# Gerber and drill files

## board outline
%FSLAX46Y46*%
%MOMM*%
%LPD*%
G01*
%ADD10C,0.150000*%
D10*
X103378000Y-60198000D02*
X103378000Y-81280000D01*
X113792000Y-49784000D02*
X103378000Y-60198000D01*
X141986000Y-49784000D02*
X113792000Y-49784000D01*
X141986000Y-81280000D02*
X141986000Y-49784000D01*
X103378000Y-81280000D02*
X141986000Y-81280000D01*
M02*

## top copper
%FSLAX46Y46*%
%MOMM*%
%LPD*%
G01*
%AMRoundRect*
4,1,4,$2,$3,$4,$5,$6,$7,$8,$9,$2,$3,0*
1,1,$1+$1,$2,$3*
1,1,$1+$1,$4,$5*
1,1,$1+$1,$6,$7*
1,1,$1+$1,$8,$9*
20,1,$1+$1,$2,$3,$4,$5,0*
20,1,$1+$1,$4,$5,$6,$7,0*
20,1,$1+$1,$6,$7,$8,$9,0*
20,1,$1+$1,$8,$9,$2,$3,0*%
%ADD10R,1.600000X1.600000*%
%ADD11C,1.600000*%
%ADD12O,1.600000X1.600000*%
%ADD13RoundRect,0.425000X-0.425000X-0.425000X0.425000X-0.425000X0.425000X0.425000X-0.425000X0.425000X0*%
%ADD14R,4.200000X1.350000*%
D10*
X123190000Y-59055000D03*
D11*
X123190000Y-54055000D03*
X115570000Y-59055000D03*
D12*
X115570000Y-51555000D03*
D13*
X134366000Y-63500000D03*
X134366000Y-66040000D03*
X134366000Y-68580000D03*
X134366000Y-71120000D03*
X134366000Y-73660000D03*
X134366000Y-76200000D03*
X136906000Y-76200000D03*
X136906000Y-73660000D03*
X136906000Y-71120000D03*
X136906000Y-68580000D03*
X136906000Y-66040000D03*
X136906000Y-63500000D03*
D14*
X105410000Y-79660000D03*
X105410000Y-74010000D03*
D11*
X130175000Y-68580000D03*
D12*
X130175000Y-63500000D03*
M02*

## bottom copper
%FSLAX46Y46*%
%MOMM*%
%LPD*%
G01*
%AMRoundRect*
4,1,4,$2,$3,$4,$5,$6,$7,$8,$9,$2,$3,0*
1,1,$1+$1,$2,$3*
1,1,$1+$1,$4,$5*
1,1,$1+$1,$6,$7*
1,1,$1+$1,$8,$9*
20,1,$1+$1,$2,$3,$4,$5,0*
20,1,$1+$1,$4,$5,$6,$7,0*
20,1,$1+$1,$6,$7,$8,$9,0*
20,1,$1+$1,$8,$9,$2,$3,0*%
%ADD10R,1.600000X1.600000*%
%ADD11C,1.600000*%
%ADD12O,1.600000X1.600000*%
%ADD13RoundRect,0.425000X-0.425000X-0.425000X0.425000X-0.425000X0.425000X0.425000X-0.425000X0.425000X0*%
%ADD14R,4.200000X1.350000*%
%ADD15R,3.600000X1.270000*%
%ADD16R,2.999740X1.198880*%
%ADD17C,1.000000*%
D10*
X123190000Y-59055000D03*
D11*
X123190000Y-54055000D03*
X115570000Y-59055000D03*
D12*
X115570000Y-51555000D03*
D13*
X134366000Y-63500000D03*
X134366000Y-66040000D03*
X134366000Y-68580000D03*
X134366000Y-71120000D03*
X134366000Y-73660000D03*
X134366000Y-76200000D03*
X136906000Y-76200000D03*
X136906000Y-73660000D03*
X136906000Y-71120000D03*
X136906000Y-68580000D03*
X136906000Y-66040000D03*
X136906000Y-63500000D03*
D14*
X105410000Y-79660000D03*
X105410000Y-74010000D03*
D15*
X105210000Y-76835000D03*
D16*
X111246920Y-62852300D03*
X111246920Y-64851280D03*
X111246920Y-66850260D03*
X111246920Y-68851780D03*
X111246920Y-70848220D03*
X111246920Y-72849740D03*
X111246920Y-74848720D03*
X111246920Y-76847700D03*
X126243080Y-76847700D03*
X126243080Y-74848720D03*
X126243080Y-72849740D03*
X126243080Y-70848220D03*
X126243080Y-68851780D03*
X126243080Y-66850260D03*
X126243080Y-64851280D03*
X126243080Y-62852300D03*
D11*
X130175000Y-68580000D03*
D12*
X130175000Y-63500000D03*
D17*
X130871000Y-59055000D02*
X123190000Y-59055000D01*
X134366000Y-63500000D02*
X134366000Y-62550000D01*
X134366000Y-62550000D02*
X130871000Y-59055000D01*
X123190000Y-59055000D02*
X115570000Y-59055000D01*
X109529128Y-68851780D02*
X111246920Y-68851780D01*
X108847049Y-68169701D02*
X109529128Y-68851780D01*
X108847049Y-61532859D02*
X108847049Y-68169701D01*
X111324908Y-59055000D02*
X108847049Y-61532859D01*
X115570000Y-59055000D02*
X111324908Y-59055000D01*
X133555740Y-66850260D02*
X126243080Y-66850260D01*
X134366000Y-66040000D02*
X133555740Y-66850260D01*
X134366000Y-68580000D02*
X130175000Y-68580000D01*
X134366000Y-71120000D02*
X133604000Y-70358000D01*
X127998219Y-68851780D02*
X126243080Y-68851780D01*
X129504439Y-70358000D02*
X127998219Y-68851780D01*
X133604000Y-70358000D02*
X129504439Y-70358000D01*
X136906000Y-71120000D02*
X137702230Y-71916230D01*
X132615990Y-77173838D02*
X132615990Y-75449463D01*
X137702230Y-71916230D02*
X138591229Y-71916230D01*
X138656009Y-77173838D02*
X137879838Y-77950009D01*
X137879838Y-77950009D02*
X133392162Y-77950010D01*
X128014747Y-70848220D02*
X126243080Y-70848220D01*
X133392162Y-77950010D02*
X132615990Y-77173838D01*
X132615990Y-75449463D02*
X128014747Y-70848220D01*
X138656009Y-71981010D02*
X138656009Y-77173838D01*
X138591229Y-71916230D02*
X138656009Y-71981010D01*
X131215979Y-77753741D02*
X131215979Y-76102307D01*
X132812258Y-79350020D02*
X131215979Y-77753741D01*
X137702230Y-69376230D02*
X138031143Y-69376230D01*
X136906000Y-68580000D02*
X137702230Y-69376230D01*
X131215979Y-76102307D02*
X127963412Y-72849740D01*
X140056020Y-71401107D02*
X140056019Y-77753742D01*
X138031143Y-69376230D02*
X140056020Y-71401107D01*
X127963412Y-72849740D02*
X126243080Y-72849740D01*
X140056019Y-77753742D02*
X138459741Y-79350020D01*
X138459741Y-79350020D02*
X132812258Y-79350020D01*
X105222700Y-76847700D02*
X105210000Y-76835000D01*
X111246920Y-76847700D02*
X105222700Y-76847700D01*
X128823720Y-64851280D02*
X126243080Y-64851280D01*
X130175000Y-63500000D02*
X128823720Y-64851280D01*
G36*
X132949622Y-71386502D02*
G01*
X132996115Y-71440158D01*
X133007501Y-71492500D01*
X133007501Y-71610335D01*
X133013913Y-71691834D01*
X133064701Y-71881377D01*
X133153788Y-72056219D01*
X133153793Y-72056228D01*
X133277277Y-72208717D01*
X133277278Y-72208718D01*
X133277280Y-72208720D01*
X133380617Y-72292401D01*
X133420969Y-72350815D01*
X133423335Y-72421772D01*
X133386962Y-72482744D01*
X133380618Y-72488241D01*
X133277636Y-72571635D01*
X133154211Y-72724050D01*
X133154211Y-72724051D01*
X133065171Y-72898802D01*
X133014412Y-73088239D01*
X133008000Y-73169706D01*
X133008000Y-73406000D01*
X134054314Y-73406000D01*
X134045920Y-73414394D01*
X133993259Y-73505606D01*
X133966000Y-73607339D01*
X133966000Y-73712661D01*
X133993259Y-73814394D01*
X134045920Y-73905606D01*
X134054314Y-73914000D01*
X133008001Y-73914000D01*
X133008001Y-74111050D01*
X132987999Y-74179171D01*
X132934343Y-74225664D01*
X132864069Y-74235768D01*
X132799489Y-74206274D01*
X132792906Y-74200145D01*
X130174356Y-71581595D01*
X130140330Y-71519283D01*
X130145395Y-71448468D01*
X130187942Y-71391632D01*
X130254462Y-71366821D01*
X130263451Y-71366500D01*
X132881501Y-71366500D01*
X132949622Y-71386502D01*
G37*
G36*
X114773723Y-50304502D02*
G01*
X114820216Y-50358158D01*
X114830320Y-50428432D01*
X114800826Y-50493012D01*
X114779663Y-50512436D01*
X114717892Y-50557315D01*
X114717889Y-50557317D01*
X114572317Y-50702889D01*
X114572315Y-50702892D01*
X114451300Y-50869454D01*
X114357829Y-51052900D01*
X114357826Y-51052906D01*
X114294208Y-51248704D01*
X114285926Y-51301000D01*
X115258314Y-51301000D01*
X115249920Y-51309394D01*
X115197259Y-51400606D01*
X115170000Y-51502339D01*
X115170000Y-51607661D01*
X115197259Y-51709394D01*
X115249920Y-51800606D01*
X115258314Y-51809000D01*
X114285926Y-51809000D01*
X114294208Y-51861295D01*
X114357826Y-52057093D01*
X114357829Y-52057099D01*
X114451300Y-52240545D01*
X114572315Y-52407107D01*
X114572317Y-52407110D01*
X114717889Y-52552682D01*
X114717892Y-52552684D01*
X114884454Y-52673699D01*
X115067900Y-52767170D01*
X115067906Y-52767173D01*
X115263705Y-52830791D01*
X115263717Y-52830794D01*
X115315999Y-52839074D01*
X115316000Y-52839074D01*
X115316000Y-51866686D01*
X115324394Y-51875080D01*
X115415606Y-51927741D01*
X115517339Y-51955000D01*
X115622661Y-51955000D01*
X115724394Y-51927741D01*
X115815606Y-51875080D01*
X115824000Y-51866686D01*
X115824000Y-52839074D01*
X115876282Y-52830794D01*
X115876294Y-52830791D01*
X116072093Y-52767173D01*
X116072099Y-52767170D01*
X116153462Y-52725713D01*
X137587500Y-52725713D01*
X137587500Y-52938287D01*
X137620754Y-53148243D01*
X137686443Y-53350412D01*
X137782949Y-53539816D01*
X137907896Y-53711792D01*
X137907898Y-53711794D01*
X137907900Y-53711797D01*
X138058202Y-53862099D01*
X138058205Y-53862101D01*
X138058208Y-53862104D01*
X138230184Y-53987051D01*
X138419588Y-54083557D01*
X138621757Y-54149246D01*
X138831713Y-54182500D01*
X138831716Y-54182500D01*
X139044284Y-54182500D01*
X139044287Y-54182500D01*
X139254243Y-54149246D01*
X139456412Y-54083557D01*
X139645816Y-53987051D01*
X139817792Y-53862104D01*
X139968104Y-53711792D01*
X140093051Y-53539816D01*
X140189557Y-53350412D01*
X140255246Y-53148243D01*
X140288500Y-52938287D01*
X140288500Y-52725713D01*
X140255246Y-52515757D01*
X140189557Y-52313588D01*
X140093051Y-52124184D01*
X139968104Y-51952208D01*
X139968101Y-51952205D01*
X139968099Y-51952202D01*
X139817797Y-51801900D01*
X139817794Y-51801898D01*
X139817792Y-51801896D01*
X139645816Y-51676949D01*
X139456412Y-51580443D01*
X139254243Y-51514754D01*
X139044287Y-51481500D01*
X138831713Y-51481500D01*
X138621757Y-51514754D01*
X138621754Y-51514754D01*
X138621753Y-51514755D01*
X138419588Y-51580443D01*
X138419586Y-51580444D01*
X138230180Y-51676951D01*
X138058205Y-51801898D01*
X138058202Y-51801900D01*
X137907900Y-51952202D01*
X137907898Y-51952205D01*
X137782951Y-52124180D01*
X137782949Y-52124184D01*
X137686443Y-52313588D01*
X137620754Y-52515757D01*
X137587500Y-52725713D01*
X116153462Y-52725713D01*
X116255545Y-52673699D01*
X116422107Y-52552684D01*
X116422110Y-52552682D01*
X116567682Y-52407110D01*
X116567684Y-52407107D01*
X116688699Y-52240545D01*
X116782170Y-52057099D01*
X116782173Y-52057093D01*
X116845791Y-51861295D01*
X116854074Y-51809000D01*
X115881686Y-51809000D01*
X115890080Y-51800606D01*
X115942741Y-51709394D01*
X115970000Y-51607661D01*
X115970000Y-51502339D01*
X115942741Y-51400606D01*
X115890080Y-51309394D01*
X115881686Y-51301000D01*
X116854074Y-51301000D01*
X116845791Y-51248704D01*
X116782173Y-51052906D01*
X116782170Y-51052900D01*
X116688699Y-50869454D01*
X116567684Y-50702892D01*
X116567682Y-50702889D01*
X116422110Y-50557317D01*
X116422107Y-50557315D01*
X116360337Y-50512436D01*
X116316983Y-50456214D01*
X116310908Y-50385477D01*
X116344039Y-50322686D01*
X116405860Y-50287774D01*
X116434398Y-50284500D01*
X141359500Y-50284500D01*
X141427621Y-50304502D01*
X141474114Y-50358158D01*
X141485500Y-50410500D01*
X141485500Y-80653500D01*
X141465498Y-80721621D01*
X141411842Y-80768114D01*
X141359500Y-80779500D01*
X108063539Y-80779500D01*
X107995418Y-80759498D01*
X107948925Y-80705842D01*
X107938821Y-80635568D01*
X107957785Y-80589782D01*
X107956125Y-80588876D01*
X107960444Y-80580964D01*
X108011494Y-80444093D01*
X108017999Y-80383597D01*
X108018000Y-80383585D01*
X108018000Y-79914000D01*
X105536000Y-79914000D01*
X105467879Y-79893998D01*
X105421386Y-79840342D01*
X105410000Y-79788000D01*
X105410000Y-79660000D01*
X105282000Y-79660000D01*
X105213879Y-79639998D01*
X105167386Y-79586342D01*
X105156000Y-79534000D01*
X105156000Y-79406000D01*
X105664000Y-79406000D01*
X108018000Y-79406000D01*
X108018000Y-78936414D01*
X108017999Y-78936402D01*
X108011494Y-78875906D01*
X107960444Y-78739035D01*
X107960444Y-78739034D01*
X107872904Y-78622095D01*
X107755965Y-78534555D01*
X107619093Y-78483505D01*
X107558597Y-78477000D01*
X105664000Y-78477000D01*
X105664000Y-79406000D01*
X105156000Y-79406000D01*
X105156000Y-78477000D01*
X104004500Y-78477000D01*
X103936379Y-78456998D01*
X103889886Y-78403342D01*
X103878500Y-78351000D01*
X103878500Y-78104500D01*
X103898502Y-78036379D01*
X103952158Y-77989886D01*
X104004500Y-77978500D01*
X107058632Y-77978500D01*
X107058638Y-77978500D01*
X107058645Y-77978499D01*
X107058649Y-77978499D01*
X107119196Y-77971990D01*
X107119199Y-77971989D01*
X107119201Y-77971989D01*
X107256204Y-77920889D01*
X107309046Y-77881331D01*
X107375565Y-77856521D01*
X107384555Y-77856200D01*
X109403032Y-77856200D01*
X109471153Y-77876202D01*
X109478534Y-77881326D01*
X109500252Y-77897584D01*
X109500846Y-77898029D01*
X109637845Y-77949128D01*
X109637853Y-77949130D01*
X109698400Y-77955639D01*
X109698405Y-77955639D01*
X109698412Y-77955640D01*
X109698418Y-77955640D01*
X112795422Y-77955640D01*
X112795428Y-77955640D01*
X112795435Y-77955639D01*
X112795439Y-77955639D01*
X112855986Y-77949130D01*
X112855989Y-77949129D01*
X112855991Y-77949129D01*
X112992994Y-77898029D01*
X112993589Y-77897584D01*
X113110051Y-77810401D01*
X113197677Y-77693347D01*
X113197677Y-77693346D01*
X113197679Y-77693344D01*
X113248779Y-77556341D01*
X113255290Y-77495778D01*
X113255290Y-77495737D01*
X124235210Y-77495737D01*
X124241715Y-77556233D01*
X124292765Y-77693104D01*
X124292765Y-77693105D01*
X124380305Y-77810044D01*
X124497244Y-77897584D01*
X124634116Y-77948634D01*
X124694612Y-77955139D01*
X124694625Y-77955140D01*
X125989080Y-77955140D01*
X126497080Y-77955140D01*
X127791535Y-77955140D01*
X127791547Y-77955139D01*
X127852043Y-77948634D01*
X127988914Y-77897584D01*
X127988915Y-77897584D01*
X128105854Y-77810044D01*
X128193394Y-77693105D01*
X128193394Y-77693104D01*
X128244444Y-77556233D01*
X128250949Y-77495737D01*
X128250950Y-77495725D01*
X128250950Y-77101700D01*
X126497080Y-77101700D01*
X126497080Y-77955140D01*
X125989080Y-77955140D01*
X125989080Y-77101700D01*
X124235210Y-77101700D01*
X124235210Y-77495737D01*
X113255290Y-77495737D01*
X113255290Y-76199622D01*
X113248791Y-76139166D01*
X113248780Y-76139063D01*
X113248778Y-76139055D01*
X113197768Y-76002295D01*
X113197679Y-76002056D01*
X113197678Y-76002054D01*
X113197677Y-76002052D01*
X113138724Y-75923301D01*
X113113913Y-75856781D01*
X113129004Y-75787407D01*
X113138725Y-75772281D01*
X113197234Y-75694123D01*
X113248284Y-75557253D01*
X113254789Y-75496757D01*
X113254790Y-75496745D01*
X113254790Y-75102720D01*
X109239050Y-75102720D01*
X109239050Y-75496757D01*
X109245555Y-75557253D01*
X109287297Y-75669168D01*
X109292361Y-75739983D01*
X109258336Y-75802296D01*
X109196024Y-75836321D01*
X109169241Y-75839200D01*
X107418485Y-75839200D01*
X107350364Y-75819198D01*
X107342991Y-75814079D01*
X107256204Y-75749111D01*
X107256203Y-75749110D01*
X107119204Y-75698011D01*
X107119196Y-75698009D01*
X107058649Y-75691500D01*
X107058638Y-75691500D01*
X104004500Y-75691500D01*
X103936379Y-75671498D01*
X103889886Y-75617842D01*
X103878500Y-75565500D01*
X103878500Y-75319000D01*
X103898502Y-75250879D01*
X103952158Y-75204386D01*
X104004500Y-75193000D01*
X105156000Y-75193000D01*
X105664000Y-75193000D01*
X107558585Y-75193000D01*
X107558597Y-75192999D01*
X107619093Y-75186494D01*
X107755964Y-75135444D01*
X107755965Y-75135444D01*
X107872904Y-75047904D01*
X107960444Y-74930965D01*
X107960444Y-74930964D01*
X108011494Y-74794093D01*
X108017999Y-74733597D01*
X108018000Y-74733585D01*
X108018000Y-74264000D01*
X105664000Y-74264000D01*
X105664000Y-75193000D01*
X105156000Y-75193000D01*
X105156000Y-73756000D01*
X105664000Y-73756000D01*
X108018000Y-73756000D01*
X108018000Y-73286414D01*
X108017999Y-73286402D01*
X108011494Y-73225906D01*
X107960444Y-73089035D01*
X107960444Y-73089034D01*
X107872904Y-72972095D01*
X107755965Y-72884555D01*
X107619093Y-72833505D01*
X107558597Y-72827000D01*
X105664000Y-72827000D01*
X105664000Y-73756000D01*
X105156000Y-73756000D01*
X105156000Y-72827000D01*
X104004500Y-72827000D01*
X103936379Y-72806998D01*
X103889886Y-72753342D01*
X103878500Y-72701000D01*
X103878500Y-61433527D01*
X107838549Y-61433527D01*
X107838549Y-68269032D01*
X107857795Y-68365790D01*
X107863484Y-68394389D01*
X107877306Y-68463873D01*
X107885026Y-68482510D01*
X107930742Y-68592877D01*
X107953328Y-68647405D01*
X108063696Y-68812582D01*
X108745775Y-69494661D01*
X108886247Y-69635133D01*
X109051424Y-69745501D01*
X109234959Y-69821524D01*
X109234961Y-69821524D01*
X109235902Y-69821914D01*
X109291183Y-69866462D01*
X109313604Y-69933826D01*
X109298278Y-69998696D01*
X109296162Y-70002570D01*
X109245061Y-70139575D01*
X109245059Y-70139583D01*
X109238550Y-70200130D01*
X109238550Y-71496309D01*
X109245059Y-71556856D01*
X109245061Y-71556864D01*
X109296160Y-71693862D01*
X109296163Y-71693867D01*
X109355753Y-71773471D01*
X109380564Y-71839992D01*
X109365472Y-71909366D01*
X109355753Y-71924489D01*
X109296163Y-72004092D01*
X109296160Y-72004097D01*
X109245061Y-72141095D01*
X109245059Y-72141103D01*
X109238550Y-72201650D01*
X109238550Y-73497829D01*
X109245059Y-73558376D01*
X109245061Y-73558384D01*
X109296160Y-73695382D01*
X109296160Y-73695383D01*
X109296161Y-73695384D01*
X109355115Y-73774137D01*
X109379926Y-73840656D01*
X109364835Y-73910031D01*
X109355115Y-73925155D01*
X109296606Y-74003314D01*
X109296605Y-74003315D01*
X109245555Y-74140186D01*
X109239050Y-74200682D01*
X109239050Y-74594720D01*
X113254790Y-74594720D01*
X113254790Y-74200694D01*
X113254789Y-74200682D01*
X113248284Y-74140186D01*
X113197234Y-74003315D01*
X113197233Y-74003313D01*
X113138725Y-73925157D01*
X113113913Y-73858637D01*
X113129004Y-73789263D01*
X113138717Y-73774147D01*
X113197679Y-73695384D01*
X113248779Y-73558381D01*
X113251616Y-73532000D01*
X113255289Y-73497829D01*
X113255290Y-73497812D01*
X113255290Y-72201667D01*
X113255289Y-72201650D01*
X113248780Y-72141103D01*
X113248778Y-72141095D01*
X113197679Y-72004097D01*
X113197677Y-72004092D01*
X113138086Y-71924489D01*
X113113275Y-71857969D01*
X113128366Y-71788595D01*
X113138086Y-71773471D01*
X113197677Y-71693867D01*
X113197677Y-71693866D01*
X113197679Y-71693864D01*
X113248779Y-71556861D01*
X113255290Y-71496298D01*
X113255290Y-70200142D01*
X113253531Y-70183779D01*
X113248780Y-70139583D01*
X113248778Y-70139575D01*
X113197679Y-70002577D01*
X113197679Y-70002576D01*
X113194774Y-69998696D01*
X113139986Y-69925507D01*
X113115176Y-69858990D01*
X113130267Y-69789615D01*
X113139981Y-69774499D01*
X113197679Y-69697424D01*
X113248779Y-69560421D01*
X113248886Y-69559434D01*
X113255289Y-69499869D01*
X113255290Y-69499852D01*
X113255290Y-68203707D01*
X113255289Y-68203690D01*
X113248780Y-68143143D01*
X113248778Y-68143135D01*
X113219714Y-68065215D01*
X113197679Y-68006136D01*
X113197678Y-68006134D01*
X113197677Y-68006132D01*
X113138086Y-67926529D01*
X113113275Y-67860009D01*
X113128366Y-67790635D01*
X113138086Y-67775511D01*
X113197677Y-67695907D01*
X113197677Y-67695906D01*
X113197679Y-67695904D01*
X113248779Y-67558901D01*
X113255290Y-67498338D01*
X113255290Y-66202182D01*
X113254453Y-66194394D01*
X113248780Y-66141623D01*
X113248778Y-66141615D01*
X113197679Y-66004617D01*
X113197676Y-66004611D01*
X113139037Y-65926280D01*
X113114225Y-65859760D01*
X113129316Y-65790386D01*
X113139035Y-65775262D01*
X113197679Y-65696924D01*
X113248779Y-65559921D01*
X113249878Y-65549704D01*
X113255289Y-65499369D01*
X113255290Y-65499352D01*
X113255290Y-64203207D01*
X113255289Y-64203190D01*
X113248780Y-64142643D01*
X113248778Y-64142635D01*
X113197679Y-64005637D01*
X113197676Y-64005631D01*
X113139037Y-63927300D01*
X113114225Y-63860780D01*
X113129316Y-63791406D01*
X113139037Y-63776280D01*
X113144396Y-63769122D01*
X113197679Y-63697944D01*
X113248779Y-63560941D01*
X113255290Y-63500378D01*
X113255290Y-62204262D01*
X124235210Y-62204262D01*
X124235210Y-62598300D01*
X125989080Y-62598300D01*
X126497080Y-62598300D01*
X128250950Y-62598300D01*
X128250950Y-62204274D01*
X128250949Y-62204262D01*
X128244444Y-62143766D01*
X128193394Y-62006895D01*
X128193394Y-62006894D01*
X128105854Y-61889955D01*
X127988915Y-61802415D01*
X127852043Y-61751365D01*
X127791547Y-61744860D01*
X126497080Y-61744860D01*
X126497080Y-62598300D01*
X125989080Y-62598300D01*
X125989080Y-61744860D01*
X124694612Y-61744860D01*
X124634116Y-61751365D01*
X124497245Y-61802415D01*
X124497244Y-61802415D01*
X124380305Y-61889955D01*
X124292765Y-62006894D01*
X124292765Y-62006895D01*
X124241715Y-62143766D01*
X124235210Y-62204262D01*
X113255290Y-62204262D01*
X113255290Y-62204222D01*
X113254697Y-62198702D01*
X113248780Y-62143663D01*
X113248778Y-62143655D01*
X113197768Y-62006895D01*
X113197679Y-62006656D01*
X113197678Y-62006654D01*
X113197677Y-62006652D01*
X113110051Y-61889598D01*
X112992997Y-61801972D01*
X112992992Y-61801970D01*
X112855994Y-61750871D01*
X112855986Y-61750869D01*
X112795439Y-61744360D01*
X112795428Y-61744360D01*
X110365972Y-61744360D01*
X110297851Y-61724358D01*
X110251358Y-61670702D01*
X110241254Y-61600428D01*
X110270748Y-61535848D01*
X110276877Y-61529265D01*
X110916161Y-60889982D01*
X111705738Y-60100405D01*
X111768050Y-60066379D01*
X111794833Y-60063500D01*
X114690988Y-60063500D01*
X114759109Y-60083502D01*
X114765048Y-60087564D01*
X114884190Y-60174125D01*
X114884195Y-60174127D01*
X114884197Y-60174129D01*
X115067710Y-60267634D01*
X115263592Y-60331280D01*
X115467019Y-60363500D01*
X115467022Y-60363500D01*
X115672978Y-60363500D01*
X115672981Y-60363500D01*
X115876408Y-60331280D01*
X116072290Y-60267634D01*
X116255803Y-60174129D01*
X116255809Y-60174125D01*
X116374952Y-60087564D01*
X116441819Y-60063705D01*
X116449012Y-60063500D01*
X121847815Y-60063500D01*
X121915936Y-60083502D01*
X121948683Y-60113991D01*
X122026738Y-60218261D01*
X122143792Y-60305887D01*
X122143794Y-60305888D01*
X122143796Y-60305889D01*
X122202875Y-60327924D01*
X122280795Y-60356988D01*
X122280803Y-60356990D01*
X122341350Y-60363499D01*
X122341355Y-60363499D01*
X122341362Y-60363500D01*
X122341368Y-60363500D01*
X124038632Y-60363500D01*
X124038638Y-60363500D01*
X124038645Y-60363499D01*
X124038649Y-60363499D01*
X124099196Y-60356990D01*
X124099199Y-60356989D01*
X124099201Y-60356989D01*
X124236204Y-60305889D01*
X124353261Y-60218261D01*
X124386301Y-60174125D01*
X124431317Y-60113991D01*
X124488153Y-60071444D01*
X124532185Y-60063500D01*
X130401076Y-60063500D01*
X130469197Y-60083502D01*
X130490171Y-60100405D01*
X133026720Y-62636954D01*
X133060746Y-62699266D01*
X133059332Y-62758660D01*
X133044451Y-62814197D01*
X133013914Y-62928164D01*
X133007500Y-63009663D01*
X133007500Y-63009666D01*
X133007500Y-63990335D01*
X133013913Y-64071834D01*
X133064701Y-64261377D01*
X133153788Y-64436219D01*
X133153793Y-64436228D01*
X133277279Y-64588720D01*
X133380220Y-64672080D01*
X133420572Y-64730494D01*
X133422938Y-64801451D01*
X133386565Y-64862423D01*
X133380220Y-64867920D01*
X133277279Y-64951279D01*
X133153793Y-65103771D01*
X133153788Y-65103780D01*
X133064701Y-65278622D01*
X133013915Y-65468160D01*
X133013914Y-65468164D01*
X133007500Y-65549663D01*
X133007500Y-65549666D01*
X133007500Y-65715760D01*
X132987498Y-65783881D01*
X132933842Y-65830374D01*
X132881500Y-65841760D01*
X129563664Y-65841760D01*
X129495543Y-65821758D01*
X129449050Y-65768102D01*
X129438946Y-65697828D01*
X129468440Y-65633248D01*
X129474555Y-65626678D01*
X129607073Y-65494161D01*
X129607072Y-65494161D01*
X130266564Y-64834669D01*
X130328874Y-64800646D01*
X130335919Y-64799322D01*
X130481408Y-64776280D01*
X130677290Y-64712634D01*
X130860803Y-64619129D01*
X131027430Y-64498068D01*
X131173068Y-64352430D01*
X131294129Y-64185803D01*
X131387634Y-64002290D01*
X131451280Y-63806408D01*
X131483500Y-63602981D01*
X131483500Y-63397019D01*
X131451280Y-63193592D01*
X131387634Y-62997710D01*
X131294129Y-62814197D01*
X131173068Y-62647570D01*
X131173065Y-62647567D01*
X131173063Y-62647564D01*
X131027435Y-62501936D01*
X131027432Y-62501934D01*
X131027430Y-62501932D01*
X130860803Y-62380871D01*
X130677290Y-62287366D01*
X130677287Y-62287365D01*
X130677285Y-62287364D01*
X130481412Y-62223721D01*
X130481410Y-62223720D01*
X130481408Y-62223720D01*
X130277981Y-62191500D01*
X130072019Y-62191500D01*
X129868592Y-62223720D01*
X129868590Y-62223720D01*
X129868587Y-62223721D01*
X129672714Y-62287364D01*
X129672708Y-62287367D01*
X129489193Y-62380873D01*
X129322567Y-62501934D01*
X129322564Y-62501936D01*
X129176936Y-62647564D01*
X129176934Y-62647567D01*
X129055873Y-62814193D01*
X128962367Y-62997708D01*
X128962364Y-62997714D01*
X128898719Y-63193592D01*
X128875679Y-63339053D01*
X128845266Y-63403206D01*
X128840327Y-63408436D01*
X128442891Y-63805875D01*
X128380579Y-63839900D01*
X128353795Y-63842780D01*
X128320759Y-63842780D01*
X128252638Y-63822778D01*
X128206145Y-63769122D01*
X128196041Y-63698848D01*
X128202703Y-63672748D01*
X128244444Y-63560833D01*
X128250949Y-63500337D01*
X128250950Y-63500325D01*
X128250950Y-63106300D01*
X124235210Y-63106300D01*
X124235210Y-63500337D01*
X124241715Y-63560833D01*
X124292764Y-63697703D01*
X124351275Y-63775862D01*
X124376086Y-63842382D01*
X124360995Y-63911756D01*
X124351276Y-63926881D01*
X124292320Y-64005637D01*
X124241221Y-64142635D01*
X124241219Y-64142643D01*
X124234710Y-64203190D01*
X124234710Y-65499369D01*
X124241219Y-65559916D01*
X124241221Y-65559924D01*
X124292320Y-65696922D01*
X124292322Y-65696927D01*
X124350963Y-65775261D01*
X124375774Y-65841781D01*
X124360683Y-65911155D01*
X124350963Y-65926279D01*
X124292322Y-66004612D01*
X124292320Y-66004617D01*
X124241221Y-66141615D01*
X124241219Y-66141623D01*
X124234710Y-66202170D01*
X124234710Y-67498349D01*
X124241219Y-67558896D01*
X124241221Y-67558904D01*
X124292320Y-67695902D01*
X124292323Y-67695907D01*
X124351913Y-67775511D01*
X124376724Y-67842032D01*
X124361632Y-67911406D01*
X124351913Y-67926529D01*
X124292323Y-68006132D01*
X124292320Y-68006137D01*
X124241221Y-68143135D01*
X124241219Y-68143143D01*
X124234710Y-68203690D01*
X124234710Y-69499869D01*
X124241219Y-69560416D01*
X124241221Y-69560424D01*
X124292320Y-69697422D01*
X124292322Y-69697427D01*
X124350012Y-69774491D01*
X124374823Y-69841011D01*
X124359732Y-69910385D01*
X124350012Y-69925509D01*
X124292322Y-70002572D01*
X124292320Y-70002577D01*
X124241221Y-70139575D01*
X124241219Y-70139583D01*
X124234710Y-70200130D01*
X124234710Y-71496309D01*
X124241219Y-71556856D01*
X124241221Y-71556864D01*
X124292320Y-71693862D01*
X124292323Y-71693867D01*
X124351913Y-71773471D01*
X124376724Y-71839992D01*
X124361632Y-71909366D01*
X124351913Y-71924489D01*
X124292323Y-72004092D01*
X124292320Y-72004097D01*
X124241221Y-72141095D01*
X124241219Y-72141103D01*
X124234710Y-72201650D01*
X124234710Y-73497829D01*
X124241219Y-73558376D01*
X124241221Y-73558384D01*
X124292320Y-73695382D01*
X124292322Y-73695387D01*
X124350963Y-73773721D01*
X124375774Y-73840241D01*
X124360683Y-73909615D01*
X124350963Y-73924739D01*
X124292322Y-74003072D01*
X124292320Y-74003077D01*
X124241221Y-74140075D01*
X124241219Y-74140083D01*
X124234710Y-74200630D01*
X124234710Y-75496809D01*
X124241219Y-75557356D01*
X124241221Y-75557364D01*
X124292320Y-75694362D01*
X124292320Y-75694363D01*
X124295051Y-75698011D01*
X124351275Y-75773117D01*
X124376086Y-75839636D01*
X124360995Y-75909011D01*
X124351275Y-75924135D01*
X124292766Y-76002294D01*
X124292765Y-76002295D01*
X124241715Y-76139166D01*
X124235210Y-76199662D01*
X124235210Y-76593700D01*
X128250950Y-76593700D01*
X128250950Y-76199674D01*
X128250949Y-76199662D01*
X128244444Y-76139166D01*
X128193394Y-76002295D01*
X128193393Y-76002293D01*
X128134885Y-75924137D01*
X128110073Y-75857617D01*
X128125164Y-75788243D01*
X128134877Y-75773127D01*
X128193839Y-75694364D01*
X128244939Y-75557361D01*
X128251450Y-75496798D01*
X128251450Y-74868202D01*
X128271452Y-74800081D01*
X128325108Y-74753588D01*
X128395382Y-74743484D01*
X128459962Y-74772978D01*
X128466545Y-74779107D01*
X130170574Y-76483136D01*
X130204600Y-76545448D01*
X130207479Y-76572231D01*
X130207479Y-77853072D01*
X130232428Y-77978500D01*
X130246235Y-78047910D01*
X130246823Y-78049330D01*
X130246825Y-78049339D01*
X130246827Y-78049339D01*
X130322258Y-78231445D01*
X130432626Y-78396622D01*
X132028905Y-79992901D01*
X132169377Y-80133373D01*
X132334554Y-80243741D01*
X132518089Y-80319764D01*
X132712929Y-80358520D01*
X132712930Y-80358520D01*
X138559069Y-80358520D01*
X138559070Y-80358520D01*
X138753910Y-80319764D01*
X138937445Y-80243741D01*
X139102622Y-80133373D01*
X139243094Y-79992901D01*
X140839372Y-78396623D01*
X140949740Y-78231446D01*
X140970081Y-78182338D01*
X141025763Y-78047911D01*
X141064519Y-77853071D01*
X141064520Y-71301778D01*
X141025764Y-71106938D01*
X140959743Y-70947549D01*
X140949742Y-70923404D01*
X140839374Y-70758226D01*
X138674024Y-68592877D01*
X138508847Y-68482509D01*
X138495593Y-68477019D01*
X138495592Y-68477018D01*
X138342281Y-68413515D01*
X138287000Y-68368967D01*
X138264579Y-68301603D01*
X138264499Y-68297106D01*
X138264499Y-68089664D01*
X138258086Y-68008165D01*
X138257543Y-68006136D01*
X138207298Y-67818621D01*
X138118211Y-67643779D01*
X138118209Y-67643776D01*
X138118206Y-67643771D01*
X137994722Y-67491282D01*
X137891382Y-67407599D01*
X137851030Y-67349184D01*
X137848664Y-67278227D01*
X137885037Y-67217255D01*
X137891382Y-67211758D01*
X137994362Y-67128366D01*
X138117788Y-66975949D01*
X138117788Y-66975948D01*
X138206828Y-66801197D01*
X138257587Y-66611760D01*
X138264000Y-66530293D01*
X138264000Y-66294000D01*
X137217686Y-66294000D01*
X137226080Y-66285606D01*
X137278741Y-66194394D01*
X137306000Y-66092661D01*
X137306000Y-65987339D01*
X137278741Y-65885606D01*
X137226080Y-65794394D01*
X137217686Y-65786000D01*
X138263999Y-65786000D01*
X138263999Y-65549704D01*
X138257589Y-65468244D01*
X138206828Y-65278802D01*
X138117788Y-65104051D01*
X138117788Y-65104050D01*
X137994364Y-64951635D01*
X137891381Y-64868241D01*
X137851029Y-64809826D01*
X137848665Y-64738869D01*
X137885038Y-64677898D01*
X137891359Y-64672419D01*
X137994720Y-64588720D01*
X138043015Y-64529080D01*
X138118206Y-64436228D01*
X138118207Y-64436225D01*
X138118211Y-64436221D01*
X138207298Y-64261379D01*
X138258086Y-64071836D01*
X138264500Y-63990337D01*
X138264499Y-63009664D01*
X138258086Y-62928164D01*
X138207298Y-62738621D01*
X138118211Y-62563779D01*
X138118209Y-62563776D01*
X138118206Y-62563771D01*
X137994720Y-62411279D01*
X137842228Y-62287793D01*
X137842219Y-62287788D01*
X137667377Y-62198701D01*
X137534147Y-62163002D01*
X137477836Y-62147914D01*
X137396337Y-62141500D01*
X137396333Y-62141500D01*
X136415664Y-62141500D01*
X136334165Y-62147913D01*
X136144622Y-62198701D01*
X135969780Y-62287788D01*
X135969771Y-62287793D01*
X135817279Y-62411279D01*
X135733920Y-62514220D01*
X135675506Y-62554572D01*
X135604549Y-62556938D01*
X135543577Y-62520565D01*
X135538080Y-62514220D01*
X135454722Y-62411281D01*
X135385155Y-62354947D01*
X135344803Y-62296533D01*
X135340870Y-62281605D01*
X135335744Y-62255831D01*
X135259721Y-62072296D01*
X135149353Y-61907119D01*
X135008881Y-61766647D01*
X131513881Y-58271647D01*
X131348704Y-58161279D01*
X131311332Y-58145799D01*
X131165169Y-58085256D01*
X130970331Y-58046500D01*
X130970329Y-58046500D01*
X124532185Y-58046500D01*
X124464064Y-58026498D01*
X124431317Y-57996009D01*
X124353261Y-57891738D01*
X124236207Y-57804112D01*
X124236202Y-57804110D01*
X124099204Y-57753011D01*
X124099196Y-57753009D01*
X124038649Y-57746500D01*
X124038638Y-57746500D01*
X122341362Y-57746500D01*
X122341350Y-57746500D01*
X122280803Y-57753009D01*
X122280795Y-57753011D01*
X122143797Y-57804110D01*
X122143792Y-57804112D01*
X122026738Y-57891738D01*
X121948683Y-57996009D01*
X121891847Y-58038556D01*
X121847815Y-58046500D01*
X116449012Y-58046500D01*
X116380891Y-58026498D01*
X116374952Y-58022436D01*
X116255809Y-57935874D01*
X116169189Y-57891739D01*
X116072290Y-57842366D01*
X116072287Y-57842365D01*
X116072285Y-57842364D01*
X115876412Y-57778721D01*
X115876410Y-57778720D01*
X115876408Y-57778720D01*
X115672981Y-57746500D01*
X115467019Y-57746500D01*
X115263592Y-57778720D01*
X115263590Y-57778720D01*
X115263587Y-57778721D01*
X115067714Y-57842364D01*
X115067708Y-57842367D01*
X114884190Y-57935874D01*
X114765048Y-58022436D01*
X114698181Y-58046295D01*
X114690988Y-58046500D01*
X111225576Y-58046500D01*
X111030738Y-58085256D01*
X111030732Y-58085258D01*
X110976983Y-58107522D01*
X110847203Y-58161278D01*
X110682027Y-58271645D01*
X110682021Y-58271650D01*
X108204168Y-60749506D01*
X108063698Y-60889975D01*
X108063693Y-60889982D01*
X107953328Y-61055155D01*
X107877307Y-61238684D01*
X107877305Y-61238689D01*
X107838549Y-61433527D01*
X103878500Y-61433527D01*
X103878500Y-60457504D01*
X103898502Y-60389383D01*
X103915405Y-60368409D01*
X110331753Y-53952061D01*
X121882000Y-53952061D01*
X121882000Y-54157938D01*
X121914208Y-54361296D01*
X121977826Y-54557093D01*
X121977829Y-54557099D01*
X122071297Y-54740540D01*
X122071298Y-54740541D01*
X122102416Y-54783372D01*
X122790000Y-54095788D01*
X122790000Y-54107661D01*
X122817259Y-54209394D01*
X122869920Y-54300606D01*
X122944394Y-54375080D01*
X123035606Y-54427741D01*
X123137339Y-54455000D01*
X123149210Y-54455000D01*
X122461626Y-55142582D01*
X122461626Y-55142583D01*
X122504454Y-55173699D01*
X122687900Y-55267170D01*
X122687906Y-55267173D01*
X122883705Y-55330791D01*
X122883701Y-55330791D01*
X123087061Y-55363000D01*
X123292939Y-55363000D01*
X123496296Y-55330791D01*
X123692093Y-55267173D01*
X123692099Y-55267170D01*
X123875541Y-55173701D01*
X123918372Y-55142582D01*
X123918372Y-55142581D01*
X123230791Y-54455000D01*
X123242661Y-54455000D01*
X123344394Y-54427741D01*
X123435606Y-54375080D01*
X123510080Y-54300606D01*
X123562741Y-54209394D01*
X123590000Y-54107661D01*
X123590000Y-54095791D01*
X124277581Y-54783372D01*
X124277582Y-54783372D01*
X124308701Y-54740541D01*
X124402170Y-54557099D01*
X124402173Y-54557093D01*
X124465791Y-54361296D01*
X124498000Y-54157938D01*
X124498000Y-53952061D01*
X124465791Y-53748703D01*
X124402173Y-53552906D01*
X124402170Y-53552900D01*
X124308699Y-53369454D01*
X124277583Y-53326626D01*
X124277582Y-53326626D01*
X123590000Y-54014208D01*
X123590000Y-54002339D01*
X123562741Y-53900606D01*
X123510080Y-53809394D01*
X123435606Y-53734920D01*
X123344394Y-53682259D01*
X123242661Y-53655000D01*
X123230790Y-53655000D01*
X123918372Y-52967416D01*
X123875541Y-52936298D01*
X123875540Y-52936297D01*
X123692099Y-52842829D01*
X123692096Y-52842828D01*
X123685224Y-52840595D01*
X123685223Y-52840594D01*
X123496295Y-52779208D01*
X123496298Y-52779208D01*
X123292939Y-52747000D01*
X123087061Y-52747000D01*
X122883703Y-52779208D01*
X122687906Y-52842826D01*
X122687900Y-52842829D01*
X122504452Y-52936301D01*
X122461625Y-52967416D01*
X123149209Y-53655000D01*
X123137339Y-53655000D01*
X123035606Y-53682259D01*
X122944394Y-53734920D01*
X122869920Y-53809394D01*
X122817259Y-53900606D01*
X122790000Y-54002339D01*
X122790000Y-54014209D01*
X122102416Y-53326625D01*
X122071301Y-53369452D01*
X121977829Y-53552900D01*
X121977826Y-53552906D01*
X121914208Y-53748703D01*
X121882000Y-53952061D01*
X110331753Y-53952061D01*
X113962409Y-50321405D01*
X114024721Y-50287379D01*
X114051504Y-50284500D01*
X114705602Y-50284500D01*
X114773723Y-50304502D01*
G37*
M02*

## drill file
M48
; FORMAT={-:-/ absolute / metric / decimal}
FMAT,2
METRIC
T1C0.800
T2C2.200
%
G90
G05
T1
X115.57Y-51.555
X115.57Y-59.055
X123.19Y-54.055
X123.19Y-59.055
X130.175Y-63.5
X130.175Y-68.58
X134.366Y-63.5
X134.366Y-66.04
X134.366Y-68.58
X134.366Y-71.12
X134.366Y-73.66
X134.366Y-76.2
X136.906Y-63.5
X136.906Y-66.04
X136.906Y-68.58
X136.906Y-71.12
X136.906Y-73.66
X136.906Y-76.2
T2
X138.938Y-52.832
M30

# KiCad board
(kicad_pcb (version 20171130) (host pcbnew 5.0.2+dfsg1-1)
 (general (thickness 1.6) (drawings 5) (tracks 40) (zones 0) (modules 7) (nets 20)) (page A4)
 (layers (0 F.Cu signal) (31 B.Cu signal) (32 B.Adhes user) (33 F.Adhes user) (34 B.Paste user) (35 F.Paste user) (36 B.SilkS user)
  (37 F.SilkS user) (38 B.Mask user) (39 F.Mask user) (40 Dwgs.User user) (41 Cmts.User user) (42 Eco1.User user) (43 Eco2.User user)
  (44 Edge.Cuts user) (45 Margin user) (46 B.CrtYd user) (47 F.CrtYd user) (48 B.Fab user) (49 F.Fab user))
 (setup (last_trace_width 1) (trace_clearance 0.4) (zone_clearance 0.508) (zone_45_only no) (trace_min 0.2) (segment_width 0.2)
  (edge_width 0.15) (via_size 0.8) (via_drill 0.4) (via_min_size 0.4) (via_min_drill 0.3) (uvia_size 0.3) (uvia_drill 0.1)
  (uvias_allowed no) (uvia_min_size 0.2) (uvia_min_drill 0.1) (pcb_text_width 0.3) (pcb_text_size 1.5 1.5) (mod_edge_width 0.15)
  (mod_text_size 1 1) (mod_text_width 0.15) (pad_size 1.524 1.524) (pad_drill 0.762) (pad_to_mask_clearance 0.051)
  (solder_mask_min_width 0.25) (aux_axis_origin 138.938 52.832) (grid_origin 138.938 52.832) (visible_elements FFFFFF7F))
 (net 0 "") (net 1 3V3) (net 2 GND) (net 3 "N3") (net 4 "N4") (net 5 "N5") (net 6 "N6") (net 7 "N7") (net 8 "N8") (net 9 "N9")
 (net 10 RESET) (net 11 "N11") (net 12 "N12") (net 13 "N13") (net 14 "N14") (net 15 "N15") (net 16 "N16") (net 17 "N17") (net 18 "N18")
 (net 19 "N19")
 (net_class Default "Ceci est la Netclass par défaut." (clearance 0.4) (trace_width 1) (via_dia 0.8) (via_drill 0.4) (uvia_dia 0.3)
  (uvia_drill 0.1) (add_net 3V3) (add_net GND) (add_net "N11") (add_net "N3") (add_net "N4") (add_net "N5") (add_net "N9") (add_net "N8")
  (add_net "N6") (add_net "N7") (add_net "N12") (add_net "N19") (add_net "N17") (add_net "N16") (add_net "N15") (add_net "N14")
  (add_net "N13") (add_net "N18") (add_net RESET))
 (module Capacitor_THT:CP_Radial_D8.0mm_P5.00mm (layer F.Cu) (at 123.19 59.055 90)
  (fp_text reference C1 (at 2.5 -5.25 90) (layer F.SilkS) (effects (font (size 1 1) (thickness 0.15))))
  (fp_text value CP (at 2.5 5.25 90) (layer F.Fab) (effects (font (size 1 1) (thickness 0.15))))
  (pad 1 thru_hole rect (at 0 0 90) (size 1.6 1.6) (drill 0.8) (layers *.Cu *.Mask) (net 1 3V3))
  (pad 2 thru_hole circle (at 5 0 90) (size 1.6 1.6) (drill 0.8) (layers *.Cu *.Mask) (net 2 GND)))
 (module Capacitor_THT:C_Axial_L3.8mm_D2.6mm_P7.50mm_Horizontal (layer F.Cu) (at 115.57 59.055 90)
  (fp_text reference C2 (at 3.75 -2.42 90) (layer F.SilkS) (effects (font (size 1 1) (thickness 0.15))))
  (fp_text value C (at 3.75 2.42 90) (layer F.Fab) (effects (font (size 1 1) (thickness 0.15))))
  (pad 1 thru_hole circle (at 0 0 90) (size 1.6 1.6) (drill 0.8) (layers *.Cu *.Mask) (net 1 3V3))
  (pad 2 thru_hole oval (at 7.5 0 90) (size 1.6 1.6) (drill 0.8) (layers *.Cu *.Mask) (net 2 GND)))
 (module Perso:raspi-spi (layer F.Cu) (at 134.366 63.5)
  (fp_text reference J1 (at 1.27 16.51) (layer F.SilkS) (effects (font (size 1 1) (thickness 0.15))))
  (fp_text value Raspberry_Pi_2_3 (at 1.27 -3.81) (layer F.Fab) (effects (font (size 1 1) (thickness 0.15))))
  (pad 17 thru_hole roundrect (at 0 0) (size 1.7 1.7) (drill 0.8) (layers *.Cu *.Mask) (roundrect_rratio 0.25) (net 1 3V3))
  (pad 19 thru_hole roundrect (at 0 2.54) (size 1.7 1.7) (drill 0.8) (layers *.Cu *.Mask) (roundrect_rratio 0.25) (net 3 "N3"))
  (pad 21 thru_hole roundrect (at 0 5.08) (size 1.7 1.7) (drill 0.8) (layers *.Cu *.Mask) (roundrect_rratio 0.25) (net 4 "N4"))
  (pad 23 thru_hole roundrect (at 0 7.62) (size 1.7 1.7) (drill 0.8) (layers *.Cu *.Mask) (roundrect_rratio 0.25) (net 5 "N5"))
  (pad 25 thru_hole roundrect (at 0 10.16) (size 1.7 1.7) (drill 0.8) (layers *.Cu *.Mask) (roundrect_rratio 0.25) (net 2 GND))
  (pad 27 thru_hole roundrect (at 0 12.7) (size 1.7 1.7) (drill 0.8) (layers *.Cu *.Mask) (roundrect_rratio 0.25) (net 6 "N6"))
  (pad 28 thru_hole roundrect (at 2.54 12.7) (size 1.7 1.7) (drill 0.8) (layers *.Cu *.Mask) (roundrect_rratio 0.25) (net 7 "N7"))
  (pad 26 thru_hole roundrect (at 2.54 10.16) (size 1.7 1.7) (drill 0.8) (layers *.Cu *.Mask) (roundrect_rratio 0.25) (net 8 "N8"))
  (pad 24 thru_hole roundrect (at 2.54 7.62) (size 1.7 1.7) (drill 0.8) (layers *.Cu *.Mask) (roundrect_rratio 0.25) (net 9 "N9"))
  (pad 22 thru_hole roundrect (at 2.54 5.08) (size 1.7 1.7) (drill 0.8) (layers *.Cu *.Mask) (roundrect_rratio 0.25) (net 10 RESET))
  (pad 20 thru_hole roundrect (at 2.54 2.54) (size 1.7 1.7) (drill 0.8) (layers *.Cu *.Mask) (roundrect_rratio 0.25) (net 2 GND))
  (pad 18 thru_hole roundrect (at 2.54 0) (size 1.7 1.7) (drill 0.8) (layers *.Cu *.Mask) (roundrect_rratio 0.25) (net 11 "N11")))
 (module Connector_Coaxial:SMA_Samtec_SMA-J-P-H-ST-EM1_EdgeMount (layer B.Cu) (at 105.41 76.835 180)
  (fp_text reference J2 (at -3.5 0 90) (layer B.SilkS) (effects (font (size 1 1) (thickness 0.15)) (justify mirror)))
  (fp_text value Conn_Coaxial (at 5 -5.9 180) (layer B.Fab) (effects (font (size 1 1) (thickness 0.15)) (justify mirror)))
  (pad 2 smd rect (at 0 -2.825 90) (size 1.35 4.2) (layers F.Cu F.Paste F.Mask) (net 2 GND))
  (pad 2 smd rect (at 0 2.825 90) (size 1.35 4.2) (layers F.Cu F.Paste F.Mask) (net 2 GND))
  (pad 2 smd rect (at 0 -2.825 90) (size 1.35 4.2) (layers B.Cu B.Paste B.Mask) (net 2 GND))
  (pad 2 smd rect (at 0 2.825 90) (size 1.35 4.2) (layers B.Cu B.Paste B.Mask) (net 2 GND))
  (pad 1 smd rect (at 0.2 0 90) (size 1.27 3.6) (layers B.Cu B.Paste B.Mask) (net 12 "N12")))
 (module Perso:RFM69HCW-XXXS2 (layer B.Cu) (at 118.745 69.85 180)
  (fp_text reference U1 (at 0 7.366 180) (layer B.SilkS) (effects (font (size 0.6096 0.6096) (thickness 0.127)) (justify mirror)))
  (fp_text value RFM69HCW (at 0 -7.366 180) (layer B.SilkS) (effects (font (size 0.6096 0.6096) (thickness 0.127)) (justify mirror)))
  (pad 16 smd rect (at 7.49808 6.9977 180) (size 2.99974 1.19888) (layers B.Cu B.Paste B.Mask) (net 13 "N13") (solder_mask_margin 0.1016))
  (pad 15 smd rect (at 7.49808 4.99872 180) (size 2.99974 1.19888) (layers B.Cu B.Paste B.Mask) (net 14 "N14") (solder_mask_margin 0.1016))
  (pad 14 smd rect (at 7.49808 2.99974 180) (size 2.99974 1.19888) (layers B.Cu B.Paste B.Mask) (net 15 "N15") (solder_mask_margin 0.1016))
  (pad 13 smd rect (at 7.49808 0.99822 180) (size 2.99974 1.19888) (layers B.Cu B.Paste B.Mask) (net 1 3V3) (solder_mask_margin 0.1016))
  (pad 12 smd rect (at 7.49808 -0.99822 180) (size 2.99974 1.19888) (layers B.Cu B.Paste B.Mask) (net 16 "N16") (solder_mask_margin 0.1016))
  (pad 11 smd rect (at 7.49808 -2.99974 180) (size 2.99974 1.19888) (layers B.Cu B.Paste B.Mask) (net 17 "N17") (solder_mask_margin 0.1016))
  (pad 10 smd rect (at 7.49808 -4.99872 180) (size 2.99974 1.19888) (layers B.Cu B.Paste B.Mask) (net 2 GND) (solder_mask_margin 0.1016))
  (pad 9 smd rect (at 7.49808 -6.9977 180) (size 2.99974 1.19888) (layers B.Cu B.Paste B.Mask) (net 12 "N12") (solder_mask_margin 0.1016))
  (pad 8 smd rect (at -7.49808 -6.9977 180) (size 2.99974 1.19888) (layers B.Cu B.Paste B.Mask) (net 2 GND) (solder_mask_margin 0.1016))
  (pad 7 smd rect (at -7.49808 -4.99872 180) (size 2.99974 1.19888) (layers B.Cu B.Paste B.Mask) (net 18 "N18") (solder_mask_margin 0.1016))
  (pad 6 smd rect (at -7.49808 -2.99974 180) (size 2.99974 1.19888) (layers B.Cu B.Paste B.Mask) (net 10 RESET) (solder_mask_margin 0.1016))
  (pad 5 smd rect (at -7.49808 -0.99822 180) (size 2.99974 1.19888) (layers B.Cu B.Paste B.Mask) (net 9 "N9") (solder_mask_margin 0.1016))
  (pad 4 smd rect (at -7.49808 0.99822 180) (size 2.99974 1.19888) (layers B.Cu B.Paste B.Mask) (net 5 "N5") (solder_mask_margin 0.1016))
  (pad 3 smd rect (at -7.49808 2.99974 180) (size 2.99974 1.19888) (layers B.Cu B.Paste B.Mask) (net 3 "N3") (solder_mask_margin 0.1016))
  (pad 2 smd rect (at -7.49808 4.99872 180) (size 2.99974 1.19888) (layers B.Cu B.Paste B.Mask) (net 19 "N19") (solder_mask_margin 0.1016))
  (pad 1 smd rect (at -7.49808 6.9977 180) (size 2.99974 1.19888) (layers B.Cu B.Paste B.Mask) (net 2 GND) (solder_mask_margin 0.1016)))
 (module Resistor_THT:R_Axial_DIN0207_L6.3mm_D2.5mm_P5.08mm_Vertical (layer F.Cu) (at 130.175 68.58 90)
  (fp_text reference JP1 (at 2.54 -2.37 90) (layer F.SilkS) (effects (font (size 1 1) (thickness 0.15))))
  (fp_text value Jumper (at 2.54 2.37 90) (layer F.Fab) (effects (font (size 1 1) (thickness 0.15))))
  (pad 1 thru_hole circle (at 0 0 90) (size 1.6 1.6) (drill 0.8) (layers *.Cu *.Mask) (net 4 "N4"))
  (pad 2 thru_hole oval (at 5.08 0 90) (size 1.6 1.6) (drill 0.8) (layers *.Cu *.Mask) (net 19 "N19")))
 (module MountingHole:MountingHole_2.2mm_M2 (layer F.Cu) (at 138.938 52.832)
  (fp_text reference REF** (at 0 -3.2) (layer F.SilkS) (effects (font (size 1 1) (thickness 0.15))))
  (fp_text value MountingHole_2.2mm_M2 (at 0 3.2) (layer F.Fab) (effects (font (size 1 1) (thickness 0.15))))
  (pad 1 np_thru_hole circle (at 0 0) (size 2.2 2.2) (drill 2.2) (layers *.Cu *.Mask)))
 (gr_line (start 103.378 60.198) (end 103.378 81.28) (layer Edge.Cuts) (width 0.15))
 (gr_line (start 113.792 49.784) (end 103.378 60.198) (layer Edge.Cuts) (width 0.15))
 (gr_line (start 141.986 49.784) (end 113.792 49.784) (layer Edge.Cuts) (width 0.15))
 (gr_line (start 141.986 81.28) (end 141.986 49.784) (layer Edge.Cuts) (width 0.15))
 (gr_line (start 103.378 81.28) (end 141.986 81.28) (layer Edge.Cuts) (width 0.15))
 (segment (start 130.871 59.055) (end 123.19 59.055) (width 1) (layer B.Cu) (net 1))
 (segment (start 134.366 63.5) (end 134.366 62.55) (width 1) (layer B.Cu) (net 1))
 (segment (start 134.366 62.55) (end 130.871 59.055) (width 1) (layer B.Cu) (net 1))
 (segment (start 123.19 59.055) (end 115.57 59.055) (width 1) (layer B.Cu) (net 1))
 (segment (start 109.529128 68.85178) (end 111.24692 68.85178) (width 1) (layer B.Cu) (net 1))
 (segment (start 108.847049 68.169701) (end 109.529128 68.85178) (width 1) (layer B.Cu) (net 1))
 (segment (start 108.847049 61.532859) (end 108.847049 68.169701) (width 1) (layer B.Cu) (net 1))
 (segment (start 111.324908 59.055) (end 108.847049 61.532859) (width 1) (layer B.Cu) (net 1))
 (segment (start 115.57 59.055) (end 111.324908 59.055) (width 1) (layer B.Cu) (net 1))
 (segment (start 133.55574 66.85026) (end 126.24308 66.85026) (width 1) (layer B.Cu) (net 3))
 (segment (start 134.366 66.04) (end 133.55574 66.85026) (width 1) (layer B.Cu) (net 3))
 (segment (start 134.366 68.58) (end 130.175 68.58) (width 1) (layer B.Cu) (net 4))
 (segment (start 134.366 71.12) (end 133.604 70.358) (width 1) (layer B.Cu) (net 5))
 (segment (start 127.998219 68.85178) (end 126.24308 68.85178) (width 1) (layer B.Cu) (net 5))
 (segment (start 129.504439 70.358) (end 127.998219 68.85178) (width 1) (layer B.Cu) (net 5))
 (segment (start 133.604 70.358) (end 129.504439 70.358) (width 1) (layer B.Cu) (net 5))
 (segment (start 136.906 71.12) (end 137.70223 71.91623) (width 1) (layer B.Cu) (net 9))
 (segment (start 132.61599 77.173838) (end 132.61599 75.449463) (width 1) (layer B.Cu) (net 9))
 (segment (start 137.70223 71.91623) (end 138.591229 71.91623) (width 1) (layer B.Cu) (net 9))
 (segment (start 138.656009 77.173838) (end 137.879838 77.950009) (width 1) (layer B.Cu) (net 9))
 (segment (start 137.879838 77.950009) (end 133.392162 77.95001) (width 1) (layer B.Cu) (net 9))
 (segment (start 128.014747 70.84822) (end 126.24308 70.84822) (width 1) (layer B.Cu) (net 9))
 (segment (start 133.392162 77.95001) (end 132.61599 77.173838) (width 1) (layer B.Cu) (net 9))
 (segment (start 132.61599 75.449463) (end 128.014747 70.84822) (width 1) (layer B.Cu) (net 9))
 (segment (start 138.656009 71.98101) (end 138.656009 77.173838) (width 1) (layer B.Cu) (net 9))
 (segment (start 138.591229 71.91623) (end 138.656009 71.98101) (width 1) (layer B.Cu) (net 9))
 (segment (start 131.215979 77.753741) (end 131.215979 76.102307) (width 1) (layer B.Cu) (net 10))
 (segment (start 132.812258 79.35002) (end 131.215979 77.753741) (width 1) (layer B.Cu) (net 10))
 (segment (start 137.70223 69.37623) (end 138.031143 69.37623) (width 1) (layer B.Cu) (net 10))
 (segment (start 136.906 68.58) (end 137.70223 69.37623) (width 1) (layer B.Cu) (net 10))
 (segment (start 131.215979 76.102307) (end 127.963412 72.84974) (width 1) (layer B.Cu) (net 10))
 (segment (start 140.05602 71.401107) (end 140.056019 77.753742) (width 1) (layer B.Cu) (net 10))
 (segment (start 138.031143 69.37623) (end 140.05602 71.401107) (width 1) (layer B.Cu) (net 10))
 (segment (start 127.963412 72.84974) (end 126.24308 72.84974) (width 1) (layer B.Cu) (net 10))
 (segment (start 140.056019 77.753742) (end 138.459741 79.35002) (width 1) (layer B.Cu) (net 10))
 (segment (start 138.459741 79.35002) (end 132.812258 79.35002) (width 1) (layer B.Cu) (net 10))
 (segment (start 105.2227 76.8477) (end 105.21 76.835) (width 1) (layer B.Cu) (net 12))
 (segment (start 111.24692 76.8477) (end 105.2227 76.8477) (width 1) (layer B.Cu) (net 12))
 (segment (start 128.82372 64.85128) (end 126.24308 64.85128) (width 1) (layer B.Cu) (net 19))
 (segment (start 130.175 63.5) (end 128.82372 64.85128) (width 1) (layer B.Cu) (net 19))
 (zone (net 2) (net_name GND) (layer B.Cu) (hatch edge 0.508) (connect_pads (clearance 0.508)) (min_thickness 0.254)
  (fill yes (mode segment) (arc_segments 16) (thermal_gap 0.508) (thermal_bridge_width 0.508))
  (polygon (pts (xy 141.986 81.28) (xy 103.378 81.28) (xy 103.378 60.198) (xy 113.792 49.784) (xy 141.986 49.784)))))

